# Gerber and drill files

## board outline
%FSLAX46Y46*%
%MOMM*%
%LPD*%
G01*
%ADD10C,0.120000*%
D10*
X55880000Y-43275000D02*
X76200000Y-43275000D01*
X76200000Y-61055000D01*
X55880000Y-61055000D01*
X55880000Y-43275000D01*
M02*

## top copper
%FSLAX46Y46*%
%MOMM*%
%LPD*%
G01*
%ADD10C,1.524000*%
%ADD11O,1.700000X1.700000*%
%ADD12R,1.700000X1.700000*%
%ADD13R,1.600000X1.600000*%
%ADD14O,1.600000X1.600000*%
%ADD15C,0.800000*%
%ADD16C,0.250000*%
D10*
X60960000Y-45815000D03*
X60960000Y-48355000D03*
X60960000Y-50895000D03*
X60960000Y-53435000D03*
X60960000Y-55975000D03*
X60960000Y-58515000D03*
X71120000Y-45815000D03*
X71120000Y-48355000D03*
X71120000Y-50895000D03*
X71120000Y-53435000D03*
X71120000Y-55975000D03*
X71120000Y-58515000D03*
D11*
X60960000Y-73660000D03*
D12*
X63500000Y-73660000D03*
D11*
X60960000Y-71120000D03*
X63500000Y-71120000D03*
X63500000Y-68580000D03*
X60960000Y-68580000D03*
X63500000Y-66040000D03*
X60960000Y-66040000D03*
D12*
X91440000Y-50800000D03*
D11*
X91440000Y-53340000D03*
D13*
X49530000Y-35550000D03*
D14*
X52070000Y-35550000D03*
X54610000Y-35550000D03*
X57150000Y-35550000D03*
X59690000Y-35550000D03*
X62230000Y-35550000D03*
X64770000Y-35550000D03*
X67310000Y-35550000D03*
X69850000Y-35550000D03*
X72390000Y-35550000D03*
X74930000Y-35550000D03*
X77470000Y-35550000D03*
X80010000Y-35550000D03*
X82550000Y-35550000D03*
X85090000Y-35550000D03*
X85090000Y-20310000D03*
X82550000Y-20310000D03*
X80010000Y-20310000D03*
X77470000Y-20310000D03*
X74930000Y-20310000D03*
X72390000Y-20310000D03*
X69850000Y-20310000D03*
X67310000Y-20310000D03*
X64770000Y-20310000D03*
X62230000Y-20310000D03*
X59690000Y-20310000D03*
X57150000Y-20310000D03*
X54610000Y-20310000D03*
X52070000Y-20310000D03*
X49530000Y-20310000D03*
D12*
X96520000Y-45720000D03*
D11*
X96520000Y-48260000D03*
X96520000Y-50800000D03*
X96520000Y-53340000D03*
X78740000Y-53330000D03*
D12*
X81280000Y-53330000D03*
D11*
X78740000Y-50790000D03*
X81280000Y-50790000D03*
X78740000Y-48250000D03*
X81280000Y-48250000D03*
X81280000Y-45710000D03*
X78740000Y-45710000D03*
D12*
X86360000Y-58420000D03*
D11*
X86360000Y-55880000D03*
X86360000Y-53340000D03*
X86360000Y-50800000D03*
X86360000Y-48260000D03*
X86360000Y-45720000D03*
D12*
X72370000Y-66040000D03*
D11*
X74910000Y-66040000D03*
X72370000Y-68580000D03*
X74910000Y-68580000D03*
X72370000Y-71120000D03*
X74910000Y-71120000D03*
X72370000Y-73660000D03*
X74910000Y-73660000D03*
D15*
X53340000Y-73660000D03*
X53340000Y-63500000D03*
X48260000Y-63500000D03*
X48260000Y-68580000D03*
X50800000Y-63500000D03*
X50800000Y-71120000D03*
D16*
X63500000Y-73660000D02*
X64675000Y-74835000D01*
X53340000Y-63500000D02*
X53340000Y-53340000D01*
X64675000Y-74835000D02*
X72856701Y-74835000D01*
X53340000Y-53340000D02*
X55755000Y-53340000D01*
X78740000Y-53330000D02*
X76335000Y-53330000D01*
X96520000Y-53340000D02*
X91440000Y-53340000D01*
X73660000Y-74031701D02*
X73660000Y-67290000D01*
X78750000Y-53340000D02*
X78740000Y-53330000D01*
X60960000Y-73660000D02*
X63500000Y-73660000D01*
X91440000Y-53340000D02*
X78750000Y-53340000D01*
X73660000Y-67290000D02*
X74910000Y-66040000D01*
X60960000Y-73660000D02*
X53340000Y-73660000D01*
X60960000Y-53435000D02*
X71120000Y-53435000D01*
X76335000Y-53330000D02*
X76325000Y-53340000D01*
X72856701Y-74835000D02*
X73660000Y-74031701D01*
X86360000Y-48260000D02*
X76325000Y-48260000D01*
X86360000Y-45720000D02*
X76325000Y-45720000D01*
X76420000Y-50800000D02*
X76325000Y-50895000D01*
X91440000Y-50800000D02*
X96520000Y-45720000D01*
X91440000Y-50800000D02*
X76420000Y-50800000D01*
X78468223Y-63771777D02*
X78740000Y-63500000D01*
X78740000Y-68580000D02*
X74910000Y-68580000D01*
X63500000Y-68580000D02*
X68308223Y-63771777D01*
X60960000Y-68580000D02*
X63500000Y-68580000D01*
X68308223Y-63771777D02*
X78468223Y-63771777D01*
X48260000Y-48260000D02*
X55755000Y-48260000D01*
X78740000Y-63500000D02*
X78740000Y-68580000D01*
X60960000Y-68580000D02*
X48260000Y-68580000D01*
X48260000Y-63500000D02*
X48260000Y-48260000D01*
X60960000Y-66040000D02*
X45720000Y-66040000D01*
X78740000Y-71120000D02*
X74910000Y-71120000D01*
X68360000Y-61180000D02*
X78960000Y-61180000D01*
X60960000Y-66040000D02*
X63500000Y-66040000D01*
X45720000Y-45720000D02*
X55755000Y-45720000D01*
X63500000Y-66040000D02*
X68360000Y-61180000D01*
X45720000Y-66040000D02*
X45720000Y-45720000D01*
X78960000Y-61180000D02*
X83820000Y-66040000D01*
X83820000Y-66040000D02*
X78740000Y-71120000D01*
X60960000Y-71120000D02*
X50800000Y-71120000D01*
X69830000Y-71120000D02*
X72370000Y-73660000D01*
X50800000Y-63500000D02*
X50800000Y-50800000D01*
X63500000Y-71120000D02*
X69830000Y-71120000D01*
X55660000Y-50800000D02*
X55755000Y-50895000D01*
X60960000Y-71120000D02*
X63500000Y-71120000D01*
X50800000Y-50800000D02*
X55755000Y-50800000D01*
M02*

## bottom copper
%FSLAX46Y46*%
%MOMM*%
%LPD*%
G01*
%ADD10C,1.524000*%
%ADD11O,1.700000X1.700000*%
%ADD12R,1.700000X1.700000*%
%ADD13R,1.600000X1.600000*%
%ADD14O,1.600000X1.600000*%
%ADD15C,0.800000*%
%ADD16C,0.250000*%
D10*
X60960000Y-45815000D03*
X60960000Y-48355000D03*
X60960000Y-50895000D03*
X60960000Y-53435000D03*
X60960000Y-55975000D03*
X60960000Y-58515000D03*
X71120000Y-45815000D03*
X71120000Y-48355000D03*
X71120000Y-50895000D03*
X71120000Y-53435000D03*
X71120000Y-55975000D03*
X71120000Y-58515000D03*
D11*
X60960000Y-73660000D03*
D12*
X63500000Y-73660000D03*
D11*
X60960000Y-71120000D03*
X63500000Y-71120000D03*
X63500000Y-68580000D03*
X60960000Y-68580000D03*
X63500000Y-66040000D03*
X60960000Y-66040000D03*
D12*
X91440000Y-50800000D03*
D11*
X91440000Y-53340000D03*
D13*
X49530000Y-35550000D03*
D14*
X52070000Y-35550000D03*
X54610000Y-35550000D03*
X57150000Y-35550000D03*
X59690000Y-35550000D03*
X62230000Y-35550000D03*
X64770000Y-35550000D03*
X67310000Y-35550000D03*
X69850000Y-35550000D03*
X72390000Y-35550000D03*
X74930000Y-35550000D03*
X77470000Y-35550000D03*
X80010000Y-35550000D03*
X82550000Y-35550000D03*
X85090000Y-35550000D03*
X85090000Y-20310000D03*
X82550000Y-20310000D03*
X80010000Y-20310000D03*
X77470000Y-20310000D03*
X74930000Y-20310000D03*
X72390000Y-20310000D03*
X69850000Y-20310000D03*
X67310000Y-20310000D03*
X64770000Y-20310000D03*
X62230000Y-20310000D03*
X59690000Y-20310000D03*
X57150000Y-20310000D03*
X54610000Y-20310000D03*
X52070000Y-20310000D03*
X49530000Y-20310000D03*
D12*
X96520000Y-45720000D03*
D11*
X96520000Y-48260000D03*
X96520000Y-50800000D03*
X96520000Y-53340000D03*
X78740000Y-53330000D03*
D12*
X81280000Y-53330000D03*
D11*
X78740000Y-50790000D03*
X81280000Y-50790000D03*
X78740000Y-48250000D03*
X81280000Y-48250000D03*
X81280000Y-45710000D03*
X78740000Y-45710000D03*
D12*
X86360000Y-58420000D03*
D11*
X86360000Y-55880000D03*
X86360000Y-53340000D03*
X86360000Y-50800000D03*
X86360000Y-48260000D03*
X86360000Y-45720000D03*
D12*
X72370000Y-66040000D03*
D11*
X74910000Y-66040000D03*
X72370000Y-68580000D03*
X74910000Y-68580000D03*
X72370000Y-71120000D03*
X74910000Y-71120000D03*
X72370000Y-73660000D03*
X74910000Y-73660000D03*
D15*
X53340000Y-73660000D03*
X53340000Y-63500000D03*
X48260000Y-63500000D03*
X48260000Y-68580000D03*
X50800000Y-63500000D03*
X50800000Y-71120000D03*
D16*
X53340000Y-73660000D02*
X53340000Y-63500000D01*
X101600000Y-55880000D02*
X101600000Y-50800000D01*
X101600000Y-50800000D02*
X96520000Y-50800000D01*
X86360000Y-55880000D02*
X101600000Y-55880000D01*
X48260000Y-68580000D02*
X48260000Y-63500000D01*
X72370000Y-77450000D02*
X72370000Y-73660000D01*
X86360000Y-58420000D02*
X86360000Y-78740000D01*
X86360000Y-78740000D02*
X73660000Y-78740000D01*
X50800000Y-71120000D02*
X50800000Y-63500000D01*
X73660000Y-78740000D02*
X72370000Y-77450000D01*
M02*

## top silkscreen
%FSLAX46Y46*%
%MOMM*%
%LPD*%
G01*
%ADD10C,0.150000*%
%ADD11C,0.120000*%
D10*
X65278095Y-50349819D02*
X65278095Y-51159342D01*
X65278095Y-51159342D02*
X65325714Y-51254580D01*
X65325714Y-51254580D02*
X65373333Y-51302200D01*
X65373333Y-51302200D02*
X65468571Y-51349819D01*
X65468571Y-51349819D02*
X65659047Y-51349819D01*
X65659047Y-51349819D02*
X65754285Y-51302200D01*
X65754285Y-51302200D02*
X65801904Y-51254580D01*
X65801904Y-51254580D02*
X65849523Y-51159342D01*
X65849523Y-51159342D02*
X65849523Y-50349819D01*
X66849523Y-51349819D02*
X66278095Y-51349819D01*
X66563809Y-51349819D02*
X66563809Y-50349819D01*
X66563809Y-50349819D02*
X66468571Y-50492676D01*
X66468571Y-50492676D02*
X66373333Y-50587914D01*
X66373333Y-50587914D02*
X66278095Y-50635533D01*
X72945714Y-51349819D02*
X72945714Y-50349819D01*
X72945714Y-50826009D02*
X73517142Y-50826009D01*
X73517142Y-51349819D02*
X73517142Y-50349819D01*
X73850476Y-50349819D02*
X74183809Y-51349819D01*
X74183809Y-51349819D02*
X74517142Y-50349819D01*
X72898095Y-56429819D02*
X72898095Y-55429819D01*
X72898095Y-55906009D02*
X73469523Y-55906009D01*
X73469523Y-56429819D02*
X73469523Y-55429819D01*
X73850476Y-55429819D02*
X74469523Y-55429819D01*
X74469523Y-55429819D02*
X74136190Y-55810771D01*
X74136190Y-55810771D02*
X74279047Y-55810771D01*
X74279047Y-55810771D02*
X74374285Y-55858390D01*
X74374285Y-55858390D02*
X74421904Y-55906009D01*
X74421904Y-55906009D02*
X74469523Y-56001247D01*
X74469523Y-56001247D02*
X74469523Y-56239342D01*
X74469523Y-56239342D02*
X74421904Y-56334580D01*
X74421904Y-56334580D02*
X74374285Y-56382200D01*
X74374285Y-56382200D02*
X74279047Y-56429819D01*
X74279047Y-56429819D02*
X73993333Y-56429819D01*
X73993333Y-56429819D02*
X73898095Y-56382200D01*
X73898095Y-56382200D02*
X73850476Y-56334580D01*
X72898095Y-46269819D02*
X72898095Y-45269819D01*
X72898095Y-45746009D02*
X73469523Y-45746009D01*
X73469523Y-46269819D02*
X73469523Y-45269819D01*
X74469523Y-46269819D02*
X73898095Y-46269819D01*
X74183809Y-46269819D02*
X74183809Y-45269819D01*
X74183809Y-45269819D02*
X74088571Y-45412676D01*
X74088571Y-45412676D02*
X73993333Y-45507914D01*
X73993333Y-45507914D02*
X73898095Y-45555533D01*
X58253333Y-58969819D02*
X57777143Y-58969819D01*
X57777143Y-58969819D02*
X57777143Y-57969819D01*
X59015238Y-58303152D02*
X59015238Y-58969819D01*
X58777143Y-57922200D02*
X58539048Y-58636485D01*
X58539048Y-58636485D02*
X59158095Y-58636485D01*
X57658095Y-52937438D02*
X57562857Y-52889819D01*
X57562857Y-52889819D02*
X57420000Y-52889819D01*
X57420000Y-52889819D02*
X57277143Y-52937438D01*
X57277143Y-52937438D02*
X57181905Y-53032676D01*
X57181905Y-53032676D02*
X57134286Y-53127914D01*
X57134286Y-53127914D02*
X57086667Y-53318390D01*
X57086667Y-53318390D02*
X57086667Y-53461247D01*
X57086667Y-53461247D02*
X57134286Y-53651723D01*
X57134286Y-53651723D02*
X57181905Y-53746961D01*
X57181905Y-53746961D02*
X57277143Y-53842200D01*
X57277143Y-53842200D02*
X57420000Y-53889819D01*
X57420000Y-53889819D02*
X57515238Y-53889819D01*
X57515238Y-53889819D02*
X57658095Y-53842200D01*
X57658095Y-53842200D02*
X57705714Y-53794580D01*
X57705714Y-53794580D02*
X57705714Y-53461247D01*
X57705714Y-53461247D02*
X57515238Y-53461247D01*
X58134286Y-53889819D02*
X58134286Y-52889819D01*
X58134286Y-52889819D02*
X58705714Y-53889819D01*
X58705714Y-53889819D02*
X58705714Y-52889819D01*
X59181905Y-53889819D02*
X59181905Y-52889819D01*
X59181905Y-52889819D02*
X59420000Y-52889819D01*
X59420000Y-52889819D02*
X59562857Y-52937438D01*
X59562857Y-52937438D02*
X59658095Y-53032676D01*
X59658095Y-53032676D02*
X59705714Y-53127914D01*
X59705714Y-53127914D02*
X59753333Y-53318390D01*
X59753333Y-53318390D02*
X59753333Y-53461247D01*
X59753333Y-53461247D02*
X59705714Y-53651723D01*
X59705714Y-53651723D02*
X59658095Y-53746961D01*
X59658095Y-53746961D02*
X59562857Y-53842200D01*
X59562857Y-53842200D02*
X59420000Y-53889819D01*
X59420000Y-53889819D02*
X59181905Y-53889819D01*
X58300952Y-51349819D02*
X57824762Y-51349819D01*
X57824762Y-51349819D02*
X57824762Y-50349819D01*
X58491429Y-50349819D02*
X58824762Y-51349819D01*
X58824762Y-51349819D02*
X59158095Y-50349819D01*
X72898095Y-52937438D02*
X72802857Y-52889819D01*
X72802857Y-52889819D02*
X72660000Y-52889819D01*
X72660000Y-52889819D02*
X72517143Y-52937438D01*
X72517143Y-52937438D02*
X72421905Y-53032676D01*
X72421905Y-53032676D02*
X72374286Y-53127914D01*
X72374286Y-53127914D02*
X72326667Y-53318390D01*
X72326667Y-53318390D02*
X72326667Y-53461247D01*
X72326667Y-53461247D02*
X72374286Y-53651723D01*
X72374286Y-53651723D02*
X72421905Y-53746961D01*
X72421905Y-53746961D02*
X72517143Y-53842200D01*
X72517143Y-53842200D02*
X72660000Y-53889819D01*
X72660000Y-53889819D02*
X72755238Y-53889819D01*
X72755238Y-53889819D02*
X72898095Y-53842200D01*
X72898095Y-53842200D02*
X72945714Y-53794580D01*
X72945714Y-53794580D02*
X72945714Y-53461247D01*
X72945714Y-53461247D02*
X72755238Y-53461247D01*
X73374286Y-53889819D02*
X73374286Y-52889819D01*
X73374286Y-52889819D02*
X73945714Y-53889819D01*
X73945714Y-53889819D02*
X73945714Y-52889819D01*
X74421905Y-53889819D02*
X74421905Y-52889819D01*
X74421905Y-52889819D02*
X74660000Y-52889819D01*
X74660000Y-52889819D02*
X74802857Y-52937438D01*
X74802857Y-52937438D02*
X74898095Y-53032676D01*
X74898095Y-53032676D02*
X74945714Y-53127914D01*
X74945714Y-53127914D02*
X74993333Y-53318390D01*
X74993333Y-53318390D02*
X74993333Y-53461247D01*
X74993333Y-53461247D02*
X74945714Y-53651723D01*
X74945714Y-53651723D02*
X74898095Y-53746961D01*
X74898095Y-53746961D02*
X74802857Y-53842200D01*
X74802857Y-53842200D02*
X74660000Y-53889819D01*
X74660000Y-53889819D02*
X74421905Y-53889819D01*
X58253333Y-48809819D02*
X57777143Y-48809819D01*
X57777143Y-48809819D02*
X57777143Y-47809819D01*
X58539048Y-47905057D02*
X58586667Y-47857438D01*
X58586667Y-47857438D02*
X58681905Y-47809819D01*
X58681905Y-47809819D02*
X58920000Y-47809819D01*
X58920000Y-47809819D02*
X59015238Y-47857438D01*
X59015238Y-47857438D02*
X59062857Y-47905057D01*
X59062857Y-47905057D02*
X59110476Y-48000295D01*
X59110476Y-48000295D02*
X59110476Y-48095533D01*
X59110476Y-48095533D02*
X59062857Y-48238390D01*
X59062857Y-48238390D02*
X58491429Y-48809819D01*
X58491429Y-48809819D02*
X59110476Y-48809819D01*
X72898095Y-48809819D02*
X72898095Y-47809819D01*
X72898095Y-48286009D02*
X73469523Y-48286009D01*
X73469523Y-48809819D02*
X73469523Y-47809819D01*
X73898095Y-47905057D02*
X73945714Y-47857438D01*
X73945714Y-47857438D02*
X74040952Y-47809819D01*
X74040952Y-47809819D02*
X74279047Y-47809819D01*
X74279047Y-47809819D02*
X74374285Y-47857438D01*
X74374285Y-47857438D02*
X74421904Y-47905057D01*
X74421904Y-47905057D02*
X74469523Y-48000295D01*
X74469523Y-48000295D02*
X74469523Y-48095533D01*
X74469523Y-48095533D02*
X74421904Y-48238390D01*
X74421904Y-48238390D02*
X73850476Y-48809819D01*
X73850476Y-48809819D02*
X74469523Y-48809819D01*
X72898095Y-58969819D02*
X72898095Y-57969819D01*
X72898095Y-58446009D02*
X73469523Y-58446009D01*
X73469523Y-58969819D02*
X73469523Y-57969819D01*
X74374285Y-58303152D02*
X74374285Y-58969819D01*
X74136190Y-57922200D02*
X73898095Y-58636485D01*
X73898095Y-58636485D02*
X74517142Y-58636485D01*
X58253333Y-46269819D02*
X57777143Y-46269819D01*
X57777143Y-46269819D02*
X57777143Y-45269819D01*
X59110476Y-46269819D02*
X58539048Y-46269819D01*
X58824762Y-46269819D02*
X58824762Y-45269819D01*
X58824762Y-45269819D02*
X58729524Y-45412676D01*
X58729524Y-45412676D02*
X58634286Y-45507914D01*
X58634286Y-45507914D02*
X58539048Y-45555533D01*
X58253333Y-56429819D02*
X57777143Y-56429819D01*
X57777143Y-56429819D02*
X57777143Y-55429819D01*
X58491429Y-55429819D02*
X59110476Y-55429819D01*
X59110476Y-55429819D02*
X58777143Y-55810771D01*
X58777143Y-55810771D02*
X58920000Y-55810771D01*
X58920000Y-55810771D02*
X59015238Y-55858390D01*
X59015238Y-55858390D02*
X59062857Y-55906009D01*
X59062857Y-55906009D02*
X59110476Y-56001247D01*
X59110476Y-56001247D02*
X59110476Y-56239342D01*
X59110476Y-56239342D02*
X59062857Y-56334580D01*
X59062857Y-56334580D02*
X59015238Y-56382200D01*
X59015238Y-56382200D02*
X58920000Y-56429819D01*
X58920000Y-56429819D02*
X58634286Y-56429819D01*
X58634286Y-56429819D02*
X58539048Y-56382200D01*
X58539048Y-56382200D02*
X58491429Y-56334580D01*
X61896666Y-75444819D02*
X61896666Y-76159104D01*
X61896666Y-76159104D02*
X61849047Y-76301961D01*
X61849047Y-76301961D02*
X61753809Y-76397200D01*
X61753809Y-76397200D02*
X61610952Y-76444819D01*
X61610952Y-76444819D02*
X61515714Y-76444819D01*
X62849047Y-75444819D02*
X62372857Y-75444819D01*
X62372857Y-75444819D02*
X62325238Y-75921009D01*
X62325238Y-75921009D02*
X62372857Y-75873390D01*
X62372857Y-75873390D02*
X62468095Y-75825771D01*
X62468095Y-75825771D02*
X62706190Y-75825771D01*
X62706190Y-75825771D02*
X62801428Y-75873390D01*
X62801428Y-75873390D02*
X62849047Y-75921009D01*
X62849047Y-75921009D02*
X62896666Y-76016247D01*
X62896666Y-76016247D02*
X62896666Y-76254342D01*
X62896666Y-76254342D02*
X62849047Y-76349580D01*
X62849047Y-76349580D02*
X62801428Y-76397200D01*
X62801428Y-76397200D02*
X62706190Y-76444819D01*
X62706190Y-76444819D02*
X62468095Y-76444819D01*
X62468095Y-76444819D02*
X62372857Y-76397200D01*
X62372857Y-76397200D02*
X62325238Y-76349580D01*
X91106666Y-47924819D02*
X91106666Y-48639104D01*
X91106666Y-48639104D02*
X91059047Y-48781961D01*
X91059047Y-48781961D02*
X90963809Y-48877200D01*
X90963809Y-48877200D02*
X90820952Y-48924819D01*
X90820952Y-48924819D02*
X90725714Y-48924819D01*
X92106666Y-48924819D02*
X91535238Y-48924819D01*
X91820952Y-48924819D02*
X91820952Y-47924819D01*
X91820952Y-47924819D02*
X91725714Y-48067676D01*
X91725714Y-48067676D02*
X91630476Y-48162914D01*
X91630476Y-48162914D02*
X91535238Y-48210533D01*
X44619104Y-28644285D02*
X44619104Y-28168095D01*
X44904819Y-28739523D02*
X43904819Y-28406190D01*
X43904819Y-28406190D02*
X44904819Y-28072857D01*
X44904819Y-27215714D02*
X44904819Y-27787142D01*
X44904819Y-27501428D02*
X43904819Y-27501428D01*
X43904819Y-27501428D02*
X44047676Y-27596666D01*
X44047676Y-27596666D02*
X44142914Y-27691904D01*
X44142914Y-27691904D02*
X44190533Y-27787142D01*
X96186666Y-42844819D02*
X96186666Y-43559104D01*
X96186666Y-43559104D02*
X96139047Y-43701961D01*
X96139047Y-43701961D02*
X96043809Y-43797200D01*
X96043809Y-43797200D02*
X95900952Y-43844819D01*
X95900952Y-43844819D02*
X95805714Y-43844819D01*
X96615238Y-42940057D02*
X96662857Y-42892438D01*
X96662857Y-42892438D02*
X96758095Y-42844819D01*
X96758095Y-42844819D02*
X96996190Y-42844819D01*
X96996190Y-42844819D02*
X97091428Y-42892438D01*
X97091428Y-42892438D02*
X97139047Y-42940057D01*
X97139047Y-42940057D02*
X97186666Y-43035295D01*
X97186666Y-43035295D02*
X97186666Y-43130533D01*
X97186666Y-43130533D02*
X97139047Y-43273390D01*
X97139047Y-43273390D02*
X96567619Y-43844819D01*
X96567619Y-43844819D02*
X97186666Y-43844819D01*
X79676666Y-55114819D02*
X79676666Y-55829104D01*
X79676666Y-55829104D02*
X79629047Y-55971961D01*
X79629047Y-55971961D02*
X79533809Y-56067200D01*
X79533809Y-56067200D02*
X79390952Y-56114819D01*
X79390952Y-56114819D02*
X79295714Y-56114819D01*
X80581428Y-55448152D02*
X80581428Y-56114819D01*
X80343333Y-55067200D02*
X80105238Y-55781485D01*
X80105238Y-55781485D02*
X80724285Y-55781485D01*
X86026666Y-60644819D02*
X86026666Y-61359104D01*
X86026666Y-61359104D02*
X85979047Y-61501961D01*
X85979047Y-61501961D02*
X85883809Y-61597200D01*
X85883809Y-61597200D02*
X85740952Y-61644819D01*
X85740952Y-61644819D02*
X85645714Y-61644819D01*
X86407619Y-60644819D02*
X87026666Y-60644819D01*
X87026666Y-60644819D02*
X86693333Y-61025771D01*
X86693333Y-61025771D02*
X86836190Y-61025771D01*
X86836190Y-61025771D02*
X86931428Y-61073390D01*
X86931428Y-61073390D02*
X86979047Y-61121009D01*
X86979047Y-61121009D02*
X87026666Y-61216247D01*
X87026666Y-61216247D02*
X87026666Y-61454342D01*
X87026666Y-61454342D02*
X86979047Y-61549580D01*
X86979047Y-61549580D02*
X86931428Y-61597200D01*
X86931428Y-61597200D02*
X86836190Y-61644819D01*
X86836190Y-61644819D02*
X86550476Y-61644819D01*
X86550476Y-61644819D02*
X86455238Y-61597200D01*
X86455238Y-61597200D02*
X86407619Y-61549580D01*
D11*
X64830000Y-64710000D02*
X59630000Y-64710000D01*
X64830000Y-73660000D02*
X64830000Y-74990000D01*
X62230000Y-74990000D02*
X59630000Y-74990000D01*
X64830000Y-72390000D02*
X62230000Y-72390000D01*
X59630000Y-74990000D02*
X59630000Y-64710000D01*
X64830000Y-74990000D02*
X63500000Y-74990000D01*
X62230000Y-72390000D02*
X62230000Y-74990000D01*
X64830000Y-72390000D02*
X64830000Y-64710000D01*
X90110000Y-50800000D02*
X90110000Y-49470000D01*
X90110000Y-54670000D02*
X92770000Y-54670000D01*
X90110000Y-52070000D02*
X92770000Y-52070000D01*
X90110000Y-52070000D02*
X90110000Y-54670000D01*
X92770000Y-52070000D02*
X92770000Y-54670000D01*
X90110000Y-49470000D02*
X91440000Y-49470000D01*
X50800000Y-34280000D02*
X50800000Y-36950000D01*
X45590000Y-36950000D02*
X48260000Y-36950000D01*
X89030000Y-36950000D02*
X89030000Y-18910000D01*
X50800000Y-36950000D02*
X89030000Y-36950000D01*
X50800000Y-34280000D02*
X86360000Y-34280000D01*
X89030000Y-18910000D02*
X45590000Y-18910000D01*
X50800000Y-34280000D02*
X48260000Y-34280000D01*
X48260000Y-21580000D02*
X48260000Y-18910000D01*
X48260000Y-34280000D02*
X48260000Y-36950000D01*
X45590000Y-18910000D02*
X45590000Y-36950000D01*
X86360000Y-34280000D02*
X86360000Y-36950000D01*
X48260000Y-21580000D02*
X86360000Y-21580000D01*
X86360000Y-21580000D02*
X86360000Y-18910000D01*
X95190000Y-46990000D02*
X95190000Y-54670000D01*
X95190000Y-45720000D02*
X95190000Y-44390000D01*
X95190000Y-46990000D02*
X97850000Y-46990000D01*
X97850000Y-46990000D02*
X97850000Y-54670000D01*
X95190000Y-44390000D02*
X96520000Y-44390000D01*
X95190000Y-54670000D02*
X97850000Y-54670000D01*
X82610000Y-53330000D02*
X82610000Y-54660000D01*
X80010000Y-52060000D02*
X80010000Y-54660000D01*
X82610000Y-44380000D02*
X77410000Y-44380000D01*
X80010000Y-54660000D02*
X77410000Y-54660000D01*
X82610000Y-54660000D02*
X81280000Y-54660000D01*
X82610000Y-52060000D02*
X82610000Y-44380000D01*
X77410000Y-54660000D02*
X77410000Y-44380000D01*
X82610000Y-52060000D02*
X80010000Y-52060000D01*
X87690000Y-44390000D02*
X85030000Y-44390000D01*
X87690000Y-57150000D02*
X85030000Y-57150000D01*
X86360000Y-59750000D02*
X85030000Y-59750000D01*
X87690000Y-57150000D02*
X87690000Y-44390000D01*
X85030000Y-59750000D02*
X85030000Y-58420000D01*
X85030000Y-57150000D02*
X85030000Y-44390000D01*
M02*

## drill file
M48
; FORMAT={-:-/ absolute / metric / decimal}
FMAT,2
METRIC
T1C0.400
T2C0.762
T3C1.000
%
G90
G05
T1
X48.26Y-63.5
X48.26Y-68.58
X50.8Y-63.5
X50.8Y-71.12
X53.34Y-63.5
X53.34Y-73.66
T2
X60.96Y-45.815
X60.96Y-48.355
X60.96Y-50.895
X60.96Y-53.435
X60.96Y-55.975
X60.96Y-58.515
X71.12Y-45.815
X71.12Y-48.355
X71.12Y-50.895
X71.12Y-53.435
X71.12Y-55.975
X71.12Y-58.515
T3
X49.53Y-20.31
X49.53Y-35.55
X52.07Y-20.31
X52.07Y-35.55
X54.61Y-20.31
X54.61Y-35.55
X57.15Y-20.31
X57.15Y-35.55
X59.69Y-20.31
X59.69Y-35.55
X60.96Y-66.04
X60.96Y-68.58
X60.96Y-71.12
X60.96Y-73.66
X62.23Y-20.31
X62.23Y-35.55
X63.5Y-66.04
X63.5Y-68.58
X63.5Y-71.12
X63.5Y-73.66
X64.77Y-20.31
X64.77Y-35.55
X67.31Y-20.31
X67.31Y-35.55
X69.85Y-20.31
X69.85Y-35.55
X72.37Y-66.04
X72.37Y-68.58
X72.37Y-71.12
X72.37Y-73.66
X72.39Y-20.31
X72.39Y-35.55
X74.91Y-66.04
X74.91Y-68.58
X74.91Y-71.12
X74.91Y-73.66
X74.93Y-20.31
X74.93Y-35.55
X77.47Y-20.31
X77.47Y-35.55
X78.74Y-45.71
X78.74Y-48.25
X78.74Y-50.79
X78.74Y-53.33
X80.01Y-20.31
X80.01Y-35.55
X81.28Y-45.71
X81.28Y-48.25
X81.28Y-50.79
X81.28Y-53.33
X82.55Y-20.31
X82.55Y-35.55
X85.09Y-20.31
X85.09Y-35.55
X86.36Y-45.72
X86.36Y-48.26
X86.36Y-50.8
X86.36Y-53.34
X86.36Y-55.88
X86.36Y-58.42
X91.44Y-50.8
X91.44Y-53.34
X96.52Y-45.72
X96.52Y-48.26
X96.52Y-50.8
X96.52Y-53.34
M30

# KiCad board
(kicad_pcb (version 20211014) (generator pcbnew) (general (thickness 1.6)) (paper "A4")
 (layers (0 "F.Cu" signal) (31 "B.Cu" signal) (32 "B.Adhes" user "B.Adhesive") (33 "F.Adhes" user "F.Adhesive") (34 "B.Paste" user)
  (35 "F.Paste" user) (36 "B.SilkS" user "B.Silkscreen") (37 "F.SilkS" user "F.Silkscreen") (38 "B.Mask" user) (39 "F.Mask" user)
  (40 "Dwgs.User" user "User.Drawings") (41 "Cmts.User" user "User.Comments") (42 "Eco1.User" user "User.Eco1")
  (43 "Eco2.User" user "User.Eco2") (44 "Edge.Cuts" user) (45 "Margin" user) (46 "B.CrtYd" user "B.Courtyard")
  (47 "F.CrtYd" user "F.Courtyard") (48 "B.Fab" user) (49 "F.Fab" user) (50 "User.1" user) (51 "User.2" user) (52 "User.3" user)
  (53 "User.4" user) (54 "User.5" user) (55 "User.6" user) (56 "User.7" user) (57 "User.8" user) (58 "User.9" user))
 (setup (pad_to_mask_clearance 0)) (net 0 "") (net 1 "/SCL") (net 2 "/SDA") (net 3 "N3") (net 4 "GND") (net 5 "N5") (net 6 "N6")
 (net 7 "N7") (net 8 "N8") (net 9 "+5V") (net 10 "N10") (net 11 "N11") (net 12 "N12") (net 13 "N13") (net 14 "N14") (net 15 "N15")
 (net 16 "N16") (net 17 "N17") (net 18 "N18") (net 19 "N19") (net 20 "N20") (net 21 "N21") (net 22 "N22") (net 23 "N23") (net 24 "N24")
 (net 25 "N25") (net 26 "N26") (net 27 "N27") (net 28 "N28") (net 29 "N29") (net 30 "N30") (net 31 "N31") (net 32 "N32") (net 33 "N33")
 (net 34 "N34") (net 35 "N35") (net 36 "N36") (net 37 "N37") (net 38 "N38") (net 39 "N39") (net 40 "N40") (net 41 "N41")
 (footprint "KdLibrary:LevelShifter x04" (layer "F.Cu") (at 58.42 40.735)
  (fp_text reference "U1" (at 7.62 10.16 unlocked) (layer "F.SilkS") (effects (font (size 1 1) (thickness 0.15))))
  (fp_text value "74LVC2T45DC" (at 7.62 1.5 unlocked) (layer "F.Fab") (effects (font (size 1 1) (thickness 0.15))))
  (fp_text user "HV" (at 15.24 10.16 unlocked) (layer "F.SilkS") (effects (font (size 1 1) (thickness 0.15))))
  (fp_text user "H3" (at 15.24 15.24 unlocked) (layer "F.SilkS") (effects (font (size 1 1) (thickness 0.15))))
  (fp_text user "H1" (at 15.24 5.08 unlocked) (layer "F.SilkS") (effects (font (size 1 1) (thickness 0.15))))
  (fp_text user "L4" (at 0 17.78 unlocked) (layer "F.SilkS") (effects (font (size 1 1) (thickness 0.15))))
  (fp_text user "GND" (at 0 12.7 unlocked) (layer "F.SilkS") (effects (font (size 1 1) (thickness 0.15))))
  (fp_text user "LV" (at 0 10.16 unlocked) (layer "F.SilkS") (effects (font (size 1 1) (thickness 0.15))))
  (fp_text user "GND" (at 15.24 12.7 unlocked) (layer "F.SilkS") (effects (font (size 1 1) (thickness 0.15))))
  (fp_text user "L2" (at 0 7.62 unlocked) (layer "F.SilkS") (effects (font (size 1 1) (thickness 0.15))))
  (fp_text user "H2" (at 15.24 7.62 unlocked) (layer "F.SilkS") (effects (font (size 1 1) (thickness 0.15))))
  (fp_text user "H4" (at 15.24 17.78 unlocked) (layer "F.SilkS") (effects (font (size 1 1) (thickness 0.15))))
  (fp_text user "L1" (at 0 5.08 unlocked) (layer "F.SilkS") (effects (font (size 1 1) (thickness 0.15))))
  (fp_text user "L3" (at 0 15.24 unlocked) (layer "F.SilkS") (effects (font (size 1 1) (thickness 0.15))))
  (fp_rect (start 17.78 20.32) (end -2.54 2.54) (layer "Edge.Cuts") (width 0.12) (fill none))
  (pad "1" thru_hole circle (at 2.54 5.08) (size 1.524 1.524) (drill 0.762) (layers *.Cu *.Mask) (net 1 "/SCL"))
  (pad "2" thru_hole circle (at 2.54 7.62) (size 1.524 1.524) (drill 0.762) (layers *.Cu *.Mask) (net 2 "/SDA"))
  (pad "3" thru_hole circle (at 2.54 10.16) (size 1.524 1.524) (drill 0.762) (layers *.Cu *.Mask) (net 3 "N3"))
  (pad "4" thru_hole circle (at 2.54 12.7) (size 1.524 1.524) (drill 0.762) (layers *.Cu *.Mask) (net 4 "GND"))
  (pad "5" thru_hole circle (at 2.54 15.24) (size 1.524 1.524) (drill 0.762) (layers *.Cu *.Mask) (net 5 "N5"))
  (pad "6" thru_hole circle (at 2.54 17.78) (size 1.524 1.524) (drill 0.762) (layers *.Cu *.Mask) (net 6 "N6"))
  (pad "7" thru_hole circle (at 12.7 5.08) (size 1.524 1.524) (drill 0.762) (layers *.Cu *.Mask) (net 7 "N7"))
  (pad "8" thru_hole circle (at 12.7 7.62) (size 1.524 1.524) (drill 0.762) (layers *.Cu *.Mask) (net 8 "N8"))
  (pad "9" thru_hole circle (at 12.7 10.16) (size 1.524 1.524) (drill 0.762) (layers *.Cu *.Mask) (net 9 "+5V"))
  (pad "10" thru_hole circle (at 12.7 12.7) (size 1.524 1.524) (drill 0.762) (layers *.Cu *.Mask) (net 4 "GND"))
  (pad "11" thru_hole circle (at 12.7 15.24) (size 1.524 1.524) (drill 0.762) (layers *.Cu *.Mask) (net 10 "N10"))
  (pad "12" thru_hole circle (at 12.7 17.78) (size 1.524 1.524) (drill 0.762) (layers *.Cu *.Mask) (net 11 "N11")))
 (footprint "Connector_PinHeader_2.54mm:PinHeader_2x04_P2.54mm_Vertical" (layer "F.Cu") (at 63.5 73.66 180)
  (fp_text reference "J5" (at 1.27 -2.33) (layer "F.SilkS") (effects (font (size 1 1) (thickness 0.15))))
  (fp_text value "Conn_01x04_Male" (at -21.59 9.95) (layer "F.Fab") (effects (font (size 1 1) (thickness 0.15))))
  (fp_line (start -1.33 8.95) (end 3.87 8.95) (layer "F.SilkS") (width 0.12))
  (fp_line (start -1.33 0) (end -1.33 -1.33) (layer "F.SilkS") (width 0.12))
  (fp_line (start 1.27 -1.33) (end 3.87 -1.33) (layer "F.SilkS") (width 0.12))
  (fp_line (start -1.33 1.27) (end 1.27 1.27) (layer "F.SilkS") (width 0.12))
  (fp_line (start 3.87 -1.33) (end 3.87 8.95) (layer "F.SilkS") (width 0.12))
  (fp_line (start -1.33 -1.33) (end 0 -1.33) (layer "F.SilkS") (width 0.12))
  (fp_line (start 1.27 1.27) (end 1.27 -1.33) (layer "F.SilkS") (width 0.12))
  (fp_line (start -1.33 1.27) (end -1.33 8.95) (layer "F.SilkS") (width 0.12))
  (pad "1" thru_hole oval (at 2.54 0 180) (size 1.7 1.7) (drill 1) (layers *.Cu *.Mask) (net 4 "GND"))
  (pad "1" thru_hole rect (at 0 0 180) (size 1.7 1.7) (drill 1) (layers *.Cu *.Mask) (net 4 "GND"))
  (pad "2" thru_hole oval (at 2.54 2.54 180) (size 1.7 1.7) (drill 1) (layers *.Cu *.Mask) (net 3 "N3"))
  (pad "2" thru_hole oval (at 0 2.54 180) (size 1.7 1.7) (drill 1) (layers *.Cu *.Mask) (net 3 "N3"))
  (pad "3" thru_hole oval (at 0 5.08 180) (size 1.7 1.7) (drill 1) (layers *.Cu *.Mask) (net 2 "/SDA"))
  (pad "3" thru_hole oval (at 2.54 5.08 180) (size 1.7 1.7) (drill 1) (layers *.Cu *.Mask) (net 2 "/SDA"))
  (pad "4" thru_hole oval (at 0 7.62 180) (size 1.7 1.7) (drill 1) (layers *.Cu *.Mask) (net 1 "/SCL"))
  (pad "4" thru_hole oval (at 2.54 7.62 180) (size 1.7 1.7) (drill 1) (layers *.Cu *.Mask) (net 1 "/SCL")))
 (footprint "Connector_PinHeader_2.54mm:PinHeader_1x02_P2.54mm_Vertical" (layer "F.Cu") (at 91.44 50.8)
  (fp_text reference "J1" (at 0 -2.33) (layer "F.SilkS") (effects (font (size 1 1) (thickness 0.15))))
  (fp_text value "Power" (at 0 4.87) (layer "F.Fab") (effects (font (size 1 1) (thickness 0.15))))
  (fp_line (start -1.33 0) (end -1.33 -1.33) (layer "F.SilkS") (width 0.12))
  (fp_line (start -1.33 3.87) (end 1.33 3.87) (layer "F.SilkS") (width 0.12))
  (fp_line (start -1.33 1.27) (end 1.33 1.27) (layer "F.SilkS") (width 0.12))
  (fp_line (start -1.33 1.27) (end -1.33 3.87) (layer "F.SilkS") (width 0.12))
  (fp_line (start 1.33 1.27) (end 1.33 3.87) (layer "F.SilkS") (width 0.12))
  (fp_line (start -1.33 -1.33) (end 0 -1.33) (layer "F.SilkS") (width 0.12))
  (pad "1" thru_hole rect (at 0 0) (size 1.7 1.7) (drill 1) (layers *.Cu *.Mask) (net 9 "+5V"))
  (pad "2" thru_hole oval (at 0 2.54) (size 1.7 1.7) (drill 1) (layers *.Cu *.Mask) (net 4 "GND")))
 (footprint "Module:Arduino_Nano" (layer "F.Cu") (at 49.53 35.55 90)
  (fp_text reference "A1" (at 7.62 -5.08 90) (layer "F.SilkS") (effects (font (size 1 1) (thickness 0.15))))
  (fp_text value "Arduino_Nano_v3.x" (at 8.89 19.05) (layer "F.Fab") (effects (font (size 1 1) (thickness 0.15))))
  (fp_line (start 1.27 1.27) (end -1.4 1.27) (layer "F.SilkS") (width 0.12))
  (fp_line (start -1.4 -3.94) (end -1.4 -1.27) (layer "F.SilkS") (width 0.12))
  (fp_line (start -1.4 39.5) (end 16.64 39.5) (layer "F.SilkS") (width 0.12))
  (fp_line (start -1.4 1.27) (end -1.4 39.5) (layer "F.SilkS") (width 0.12))
  (fp_line (start 1.27 1.27) (end 1.27 36.83) (layer "F.SilkS") (width 0.12))
  (fp_line (start 16.64 39.5) (end 16.64 -3.94) (layer "F.SilkS") (width 0.12))
  (fp_line (start 1.27 1.27) (end 1.27 -1.27) (layer "F.SilkS") (width 0.12))
  (fp_line (start 13.97 -1.27) (end 16.64 -1.27) (layer "F.SilkS") (width 0.12))
  (fp_line (start 1.27 -1.27) (end -1.4 -1.27) (layer "F.SilkS") (width 0.12))
  (fp_line (start 16.64 -3.94) (end -1.4 -3.94) (layer "F.SilkS") (width 0.12))
  (fp_line (start 1.27 36.83) (end -1.4 36.83) (layer "F.SilkS") (width 0.12))
  (fp_line (start 13.97 -1.27) (end 13.97 36.83) (layer "F.SilkS") (width 0.12))
  (fp_line (start 13.97 36.83) (end 16.64 36.83) (layer "F.SilkS") (width 0.12))
  (pad "1" thru_hole rect (at 0 0 90) (size 1.6 1.6) (drill 1) (layers *.Cu *.Mask) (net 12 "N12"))
  (pad "2" thru_hole oval (at 0 2.54 90) (size 1.6 1.6) (drill 1) (layers *.Cu *.Mask) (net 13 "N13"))
  (pad "3" thru_hole oval (at 0 5.08 90) (size 1.6 1.6) (drill 1) (layers *.Cu *.Mask) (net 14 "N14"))
  (pad "4" thru_hole oval (at 0 7.62 90) (size 1.6 1.6) (drill 1) (layers *.Cu *.Mask) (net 4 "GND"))
  (pad "5" thru_hole oval (at 0 10.16 90) (size 1.6 1.6) (drill 1) (layers *.Cu *.Mask) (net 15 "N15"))
  (pad "6" thru_hole oval (at 0 12.7 90) (size 1.6 1.6) (drill 1) (layers *.Cu *.Mask) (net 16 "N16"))
  (pad "7" thru_hole oval (at 0 15.24 90) (size 1.6 1.6) (drill 1) (layers *.Cu *.Mask) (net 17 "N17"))
  (pad "8" thru_hole oval (at 0 17.78 90) (size 1.6 1.6) (drill 1) (layers *.Cu *.Mask) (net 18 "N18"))
  (pad "9" thru_hole oval (at 0 20.32 90) (size 1.6 1.6) (drill 1) (layers *.Cu *.Mask) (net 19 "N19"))
  (pad "10" thru_hole oval (at 0 22.86 90) (size 1.6 1.6) (drill 1) (layers *.Cu *.Mask) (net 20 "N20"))
  (pad "11" thru_hole oval (at 0 25.4 90) (size 1.6 1.6) (drill 1) (layers *.Cu *.Mask) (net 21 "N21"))
  (pad "12" thru_hole oval (at 0 27.94 90) (size 1.6 1.6) (drill 1) (layers *.Cu *.Mask) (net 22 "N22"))
  (pad "13" thru_hole oval (at 0 30.48 90) (size 1.6 1.6) (drill 1) (layers *.Cu *.Mask) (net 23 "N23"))
  (pad "14" thru_hole oval (at 0 33.02 90) (size 1.6 1.6) (drill 1) (layers *.Cu *.Mask) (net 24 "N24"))
  (pad "15" thru_hole oval (at 0 35.56 90) (size 1.6 1.6) (drill 1) (layers *.Cu *.Mask) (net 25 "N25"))
  (pad "16" thru_hole oval (at 15.24 35.56 90) (size 1.6 1.6) (drill 1) (layers *.Cu *.Mask) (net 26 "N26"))
  (pad "17" thru_hole oval (at 15.24 33.02 90) (size 1.6 1.6) (drill 1) (layers *.Cu *.Mask) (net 3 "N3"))
  (pad "18" thru_hole oval (at 15.24 30.48 90) (size 1.6 1.6) (drill 1) (layers *.Cu *.Mask) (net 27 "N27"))
  (pad "19" thru_hole oval (at 15.24 27.94 90) (size 1.6 1.6) (drill 1) (layers *.Cu *.Mask) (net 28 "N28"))
  (pad "20" thru_hole oval (at 15.24 25.4 90) (size 1.6 1.6) (drill 1) (layers *.Cu *.Mask) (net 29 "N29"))
  (pad "21" thru_hole oval (at 15.24 22.86 90) (size 1.6 1.6) (drill 1) (layers *.Cu *.Mask) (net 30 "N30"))
  (pad "22" thru_hole oval (at 15.24 20.32 90) (size 1.6 1.6) (drill 1) (layers *.Cu *.Mask) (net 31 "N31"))
  (pad "23" thru_hole oval (at 15.24 17.78 90) (size 1.6 1.6) (drill 1) (layers *.Cu *.Mask) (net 8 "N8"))
  (pad "24" thru_hole oval (at 15.24 15.24 90) (size 1.6 1.6) (drill 1) (layers *.Cu *.Mask) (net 7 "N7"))
  (pad "25" thru_hole oval (at 15.24 12.7 90) (size 1.6 1.6) (drill 1) (layers *.Cu *.Mask) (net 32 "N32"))
  (pad "26" thru_hole oval (at 15.24 10.16 90) (size 1.6 1.6) (drill 1) (layers *.Cu *.Mask) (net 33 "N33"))
  (pad "27" thru_hole oval (at 15.24 7.62 90) (size 1.6 1.6) (drill 1) (layers *.Cu *.Mask) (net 9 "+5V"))
  (pad "28" thru_hole oval (at 15.24 5.08 90) (size 1.6 1.6) (drill 1) (layers *.Cu *.Mask) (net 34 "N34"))
  (pad "29" thru_hole oval (at 15.24 2.54 90) (size 1.6 1.6) (drill 1) (layers *.Cu *.Mask) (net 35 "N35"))
  (pad "30" thru_hole oval (at 15.24 0 90) (size 1.6 1.6) (drill 1) (layers *.Cu *.Mask) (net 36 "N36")))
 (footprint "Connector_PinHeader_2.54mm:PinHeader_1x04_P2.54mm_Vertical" (layer "F.Cu") (at 96.52 45.72)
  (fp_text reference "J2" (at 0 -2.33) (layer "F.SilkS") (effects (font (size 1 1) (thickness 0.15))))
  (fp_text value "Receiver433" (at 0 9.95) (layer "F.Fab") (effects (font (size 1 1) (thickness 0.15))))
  (fp_line (start -1.33 1.27) (end -1.33 8.95) (layer "F.SilkS") (width 0.12))
  (fp_line (start -1.33 0) (end -1.33 -1.33) (layer "F.SilkS") (width 0.12))
  (fp_line (start -1.33 1.27) (end 1.33 1.27) (layer "F.SilkS") (width 0.12))
  (fp_line (start 1.33 1.27) (end 1.33 8.95) (layer "F.SilkS") (width 0.12))
  (fp_line (start -1.33 -1.33) (end 0 -1.33) (layer "F.SilkS") (width 0.12))
  (fp_line (start -1.33 8.95) (end 1.33 8.95) (layer "F.SilkS") (width 0.12))
  (pad "1" thru_hole rect (at 0 0) (size 1.7 1.7) (drill 1) (layers *.Cu *.Mask) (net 9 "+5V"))
  (pad "2" thru_hole oval (at 0 2.54) (size 1.7 1.7) (drill 1) (layers *.Cu *.Mask) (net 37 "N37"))
  (pad "3" thru_hole oval (at 0 5.08) (size 1.7 1.7) (drill 1) (layers *.Cu *.Mask) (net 17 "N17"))
  (pad "4" thru_hole oval (at 0 7.62) (size 1.7 1.7) (drill 1) (layers *.Cu *.Mask) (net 4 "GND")))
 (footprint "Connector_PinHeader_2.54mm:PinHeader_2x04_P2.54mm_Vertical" (layer "F.Cu") (at 81.28 53.33 180)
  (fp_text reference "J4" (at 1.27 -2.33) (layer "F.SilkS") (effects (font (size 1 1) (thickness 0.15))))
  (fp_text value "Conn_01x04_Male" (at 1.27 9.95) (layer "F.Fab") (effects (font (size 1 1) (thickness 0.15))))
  (fp_line (start -1.33 0) (end -1.33 -1.33) (layer "F.SilkS") (width 0.12))
  (fp_line (start 1.27 1.27) (end 1.27 -1.33) (layer "F.SilkS") (width 0.12))
  (fp_line (start -1.33 8.95) (end 3.87 8.95) (layer "F.SilkS") (width 0.12))
  (fp_line (start 1.27 -1.33) (end 3.87 -1.33) (layer "F.SilkS") (width 0.12))
  (fp_line (start -1.33 -1.33) (end 0 -1.33) (layer "F.SilkS") (width 0.12))
  (fp_line (start -1.33 1.27) (end -1.33 8.95) (layer "F.SilkS") (width 0.12))
  (fp_line (start 3.87 -1.33) (end 3.87 8.95) (layer "F.SilkS") (width 0.12))
  (fp_line (start -1.33 1.27) (end 1.27 1.27) (layer "F.SilkS") (width 0.12))
  (pad "1" thru_hole oval (at 2.54 0 180) (size 1.7 1.7) (drill 1) (layers *.Cu *.Mask) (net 4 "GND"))
  (pad "1" thru_hole rect (at 0 0 180) (size 1.7 1.7) (drill 1) (layers *.Cu *.Mask) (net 4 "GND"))
  (pad "2" thru_hole oval (at 2.54 2.54 180) (size 1.7 1.7) (drill 1) (layers *.Cu *.Mask) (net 9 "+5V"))
  (pad "2" thru_hole oval (at 0 2.54 180) (size 1.7 1.7) (drill 1) (layers *.Cu *.Mask) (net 9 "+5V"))
  (pad "3" thru_hole oval (at 2.54 5.08 180) (size 1.7 1.7) (drill 1) (layers *.Cu *.Mask) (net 8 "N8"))
  (pad "3" thru_hole oval (at 0 5.08 180) (size 1.7 1.7) (drill 1) (layers *.Cu *.Mask) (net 8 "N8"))
  (pad "4" thru_hole oval (at 0 7.62 180) (size 1.7 1.7) (drill 1) (layers *.Cu *.Mask) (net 7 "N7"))
  (pad "4" thru_hole oval (at 2.54 7.62 180) (size 1.7 1.7) (drill 1) (layers *.Cu *.Mask) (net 7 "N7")))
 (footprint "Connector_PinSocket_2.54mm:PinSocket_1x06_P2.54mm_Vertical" (layer "F.Cu") (at 86.36 58.42 180)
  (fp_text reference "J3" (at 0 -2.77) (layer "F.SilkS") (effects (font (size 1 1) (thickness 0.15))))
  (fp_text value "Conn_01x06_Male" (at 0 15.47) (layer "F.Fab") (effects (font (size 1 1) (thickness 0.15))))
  (fp_line (start -1.33 14.03) (end 1.33 14.03) (layer "F.SilkS") (width 0.12))
  (fp_line (start -1.33 1.27) (end 1.33 1.27) (layer "F.SilkS") (width 0.12))
  (fp_line (start 0 -1.33) (end 1.33 -1.33) (layer "F.SilkS") (width 0.12))
  (fp_line (start -1.33 1.27) (end -1.33 14.03) (layer "F.SilkS") (width 0.12))
  (fp_line (start 1.33 -1.33) (end 1.33 0) (layer "F.SilkS") (width 0.12))
  (fp_line (start 1.33 1.27) (end 1.33 14.03) (layer "F.SilkS") (width 0.12))
  (pad "1" thru_hole rect (at 0 0 180) (size 1.7 1.7) (drill 1) (layers *.Cu *.Mask) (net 3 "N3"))
  (pad "2" thru_hole oval (at 0 2.54 180) (size 1.7 1.7) (drill 1) (layers *.Cu *.Mask) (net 17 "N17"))
  (pad "3" thru_hole oval (at 0 5.08 180) (size 1.7 1.7) (drill 1) (layers *.Cu *.Mask) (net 4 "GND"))
  (pad "4" thru_hole oval (at 0 7.62 180) (size 1.7 1.7) (drill 1) (layers *.Cu *.Mask) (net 9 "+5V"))
  (pad "5" thru_hole oval (at 0 10.16 180) (size 1.7 1.7) (drill 1) (layers *.Cu *.Mask) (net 8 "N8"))
  (pad "6" thru_hole oval (at 0 12.7 180) (size 1.7 1.7) (drill 1) (layers *.Cu *.Mask) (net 7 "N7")))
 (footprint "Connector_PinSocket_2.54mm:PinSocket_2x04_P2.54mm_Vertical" (layer "B.Cu") (at 72.37 66.04 180)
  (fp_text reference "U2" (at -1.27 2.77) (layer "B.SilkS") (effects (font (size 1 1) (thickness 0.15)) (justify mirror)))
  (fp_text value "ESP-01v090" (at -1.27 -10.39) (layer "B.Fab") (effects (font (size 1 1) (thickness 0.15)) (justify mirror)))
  (pad "1" thru_hole rect (at 0 0 180) (size 1.7 1.7) (drill 1) (layers *.Cu *.Mask) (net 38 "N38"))
  (pad "2" thru_hole oval (at -2.54 0 180) (size 1.7 1.7) (drill 1) (layers *.Cu *.Mask) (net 4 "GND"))
  (pad "3" thru_hole oval (at 0 -2.54 180) (size 1.7 1.7) (drill 1) (layers *.Cu *.Mask) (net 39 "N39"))
  (pad "4" thru_hole oval (at -2.54 -2.54 180) (size 1.7 1.7) (drill 1) (layers *.Cu *.Mask) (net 2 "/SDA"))
  (pad "5" thru_hole oval (at 0 -5.08 180) (size 1.7 1.7) (drill 1) (layers *.Cu *.Mask) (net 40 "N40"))
  (pad "6" thru_hole oval (at -2.54 -5.08 180) (size 1.7 1.7) (drill 1) (layers *.Cu *.Mask) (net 1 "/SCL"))
  (pad "7" thru_hole oval (at 0 -7.62 180) (size 1.7 1.7) (drill 1) (layers *.Cu *.Mask) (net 3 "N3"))
  (pad "8" thru_hole oval (at -2.54 -7.62 180) (size 1.7 1.7) (drill 1) (layers *.Cu *.Mask) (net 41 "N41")))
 (segment (start 63.5 73.66) (end 64.675 74.835) (width 0.25) (layer "F.Cu") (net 4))
 (segment (start 53.34 63.5) (end 53.34 53.34) (width 0.25) (layer "F.Cu") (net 4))
 (segment (start 64.675 74.835) (end 72.856701 74.835) (width 0.25) (layer "F.Cu") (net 4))
 (segment (start 53.34 53.34) (end 55.755 53.34) (width 0.25) (layer "F.Cu") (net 4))
 (segment (start 78.74 53.33) (end 76.335 53.33) (width 0.25) (layer "F.Cu") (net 4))
 (segment (start 96.52 53.34) (end 91.44 53.34) (width 0.25) (layer "F.Cu") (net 4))
 (segment (start 73.66 74.031701) (end 73.66 67.29) (width 0.25) (layer "F.Cu") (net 4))
 (segment (start 78.75 53.34) (end 78.74 53.33) (width 0.25) (layer "F.Cu") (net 4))
 (segment (start 60.96 73.66) (end 63.5 73.66) (width 0.25) (layer "F.Cu") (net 4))
 (segment (start 91.44 53.34) (end 78.75 53.34) (width 0.25) (layer "F.Cu") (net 4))
 (segment (start 73.66 67.29) (end 74.91 66.04) (width 0.25) (layer "F.Cu") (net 4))
 (segment (start 60.96 73.66) (end 53.34 73.66) (width 0.25) (layer "F.Cu") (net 4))
 (segment (start 60.96 53.435) (end 71.12 53.435) (width 0.25) (layer "F.Cu") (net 4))
 (segment (start 76.335 53.33) (end 76.325 53.34) (width 0.25) (layer "F.Cu") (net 4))
 (segment (start 72.856701 74.835) (end 73.66 74.031701) (width 0.25) (layer "F.Cu") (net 4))
 (via (at 53.34 73.66) (size 0.8) (drill 0.4) (layers "F.Cu" "B.Cu") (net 4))
 (via (at 53.34 63.5) (size 0.8) (drill 0.4) (layers "F.Cu" "B.Cu") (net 4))
 (segment (start 53.34 73.66) (end 53.34 63.5) (width 0.25) (layer "B.Cu") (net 4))
 (segment (start 101.6 55.88) (end 101.6 50.8) (width 0.25) (layer "B.Cu") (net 17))
 (segment (start 101.6 50.8) (end 96.52 50.8) (width 0.25) (layer "B.Cu") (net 17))
 (segment (start 86.36 55.88) (end 101.6 55.88) (width 0.25) (layer "B.Cu") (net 17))
 (segment (start 86.36 48.26) (end 76.325 48.26) (width 0.25) (layer "F.Cu") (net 8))
 (segment (start 86.36 45.72) (end 76.325 45.72) (width 0.25) (layer "F.Cu") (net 7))
 (segment (start 76.42 50.8) (end 76.325 50.895) (width 0.25) (layer "F.Cu") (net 9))
 (segment (start 91.44 50.8) (end 96.52 45.72) (width 0.25) (layer "F.Cu") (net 9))
 (segment (start 91.44 50.8) (end 76.42 50.8) (width 0.25) (layer "F.Cu") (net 9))
 (segment (start 78.468223 63.771777) (end 78.74 63.5) (width 0.25) (layer "F.Cu") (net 2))
 (segment (start 78.74 68.58) (end 74.91 68.58) (width 0.25) (layer "F.Cu") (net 2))
 (segment (start 63.5 68.58) (end 68.308223 63.771777) (width 0.25) (layer "F.Cu") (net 2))
 (segment (start 60.96 68.58) (end 63.5 68.58) (width 0.25) (layer "F.Cu") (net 2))
 (segment (start 68.308223 63.771777) (end 78.468223 63.771777) (width 0.25) (layer "F.Cu") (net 2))
 (segment (start 48.26 48.26) (end 55.755 48.26) (width 0.25) (layer "F.Cu") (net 2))
 (segment (start 78.74 63.5) (end 78.74 68.58) (width 0.25) (layer "F.Cu") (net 2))
 (segment (start 60.96 68.58) (end 48.26 68.58) (width 0.25) (layer "F.Cu") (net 2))
 (segment (start 48.26 63.5) (end 48.26 48.26) (width 0.25) (layer "F.Cu") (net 2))
 (via (at 48.26 63.5) (size 0.8) (drill 0.4) (layers "F.Cu" "B.Cu") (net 2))
 (via (at 48.26 68.58) (size 0.8) (drill 0.4) (layers "F.Cu" "B.Cu") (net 2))
 (segment (start 48.26 68.58) (end 48.26 63.5) (width 0.25) (layer "B.Cu") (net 2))
 (segment (start 60.96 66.04) (end 45.72 66.04) (width 0.25) (layer "F.Cu") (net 1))
 (segment (start 78.74 71.12) (end 74.91 71.12) (width 0.25) (layer "F.Cu") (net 1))
 (segment (start 68.36 61.18) (end 78.96 61.18) (width 0.25) (layer "F.Cu") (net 1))
 (segment (start 60.96 66.04) (end 63.5 66.04) (width 0.25) (layer "F.Cu") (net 1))
 (segment (start 45.72 45.72) (end 55.755 45.72) (width 0.25) (layer "F.Cu") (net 1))
 (segment (start 63.5 66.04) (end 68.36 61.18) (width 0.25) (layer "F.Cu") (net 1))
 (segment (start 45.72 66.04) (end 45.72 45.72) (width 0.25) (layer "F.Cu") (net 1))
 (segment (start 78.96 61.18) (end 83.82 66.04) (width 0.25) (layer "F.Cu") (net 1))
 (segment (start 83.82 66.04) (end 78.74 71.12) (width 0.25) (layer "F.Cu") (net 1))
 (segment (start 60.96 71.12) (end 50.8 71.12) (width 0.25) (layer "F.Cu") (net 3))
 (segment (start 69.83 71.12) (end 72.37 73.66) (width 0.25) (layer "F.Cu") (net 3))
 (segment (start 50.8 63.5) (end 50.8 50.8) (width 0.25) (layer "F.Cu") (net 3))
 (segment (start 63.5 71.12) (end 69.83 71.12) (width 0.25) (layer "F.Cu") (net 3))
 (segment (start 55.66 50.8) (end 55.755 50.895) (width 0.25) (layer "F.Cu") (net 3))
 (segment (start 60.96 71.12) (end 63.5 71.12) (width 0.25) (layer "F.Cu") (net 3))
 (segment (start 50.8 50.8) (end 55.755 50.8) (width 0.25) (layer "F.Cu") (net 3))
 (via (at 50.8 63.5) (size 0.8) (drill 0.4) (layers "F.Cu" "B.Cu") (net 3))
 (via (at 50.8 71.12) (size 0.8) (drill 0.4) (layers "F.Cu" "B.Cu") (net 3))
 (segment (start 72.37 77.45) (end 72.37 73.66) (width 0.25) (layer "B.Cu") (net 3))
 (segment (start 86.36 58.42) (end 86.36 78.74) (width 0.25) (layer "B.Cu") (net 3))
 (segment (start 86.36 78.74) (end 73.66 78.74) (width 0.25) (layer "B.Cu") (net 3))
 (segment (start 50.8 71.12) (end 50.8 63.5) (width 0.25) (layer "B.Cu") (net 3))
 (segment (start 73.66 78.74) (end 72.37 77.45) (width 0.25) (layer "B.Cu") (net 3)))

